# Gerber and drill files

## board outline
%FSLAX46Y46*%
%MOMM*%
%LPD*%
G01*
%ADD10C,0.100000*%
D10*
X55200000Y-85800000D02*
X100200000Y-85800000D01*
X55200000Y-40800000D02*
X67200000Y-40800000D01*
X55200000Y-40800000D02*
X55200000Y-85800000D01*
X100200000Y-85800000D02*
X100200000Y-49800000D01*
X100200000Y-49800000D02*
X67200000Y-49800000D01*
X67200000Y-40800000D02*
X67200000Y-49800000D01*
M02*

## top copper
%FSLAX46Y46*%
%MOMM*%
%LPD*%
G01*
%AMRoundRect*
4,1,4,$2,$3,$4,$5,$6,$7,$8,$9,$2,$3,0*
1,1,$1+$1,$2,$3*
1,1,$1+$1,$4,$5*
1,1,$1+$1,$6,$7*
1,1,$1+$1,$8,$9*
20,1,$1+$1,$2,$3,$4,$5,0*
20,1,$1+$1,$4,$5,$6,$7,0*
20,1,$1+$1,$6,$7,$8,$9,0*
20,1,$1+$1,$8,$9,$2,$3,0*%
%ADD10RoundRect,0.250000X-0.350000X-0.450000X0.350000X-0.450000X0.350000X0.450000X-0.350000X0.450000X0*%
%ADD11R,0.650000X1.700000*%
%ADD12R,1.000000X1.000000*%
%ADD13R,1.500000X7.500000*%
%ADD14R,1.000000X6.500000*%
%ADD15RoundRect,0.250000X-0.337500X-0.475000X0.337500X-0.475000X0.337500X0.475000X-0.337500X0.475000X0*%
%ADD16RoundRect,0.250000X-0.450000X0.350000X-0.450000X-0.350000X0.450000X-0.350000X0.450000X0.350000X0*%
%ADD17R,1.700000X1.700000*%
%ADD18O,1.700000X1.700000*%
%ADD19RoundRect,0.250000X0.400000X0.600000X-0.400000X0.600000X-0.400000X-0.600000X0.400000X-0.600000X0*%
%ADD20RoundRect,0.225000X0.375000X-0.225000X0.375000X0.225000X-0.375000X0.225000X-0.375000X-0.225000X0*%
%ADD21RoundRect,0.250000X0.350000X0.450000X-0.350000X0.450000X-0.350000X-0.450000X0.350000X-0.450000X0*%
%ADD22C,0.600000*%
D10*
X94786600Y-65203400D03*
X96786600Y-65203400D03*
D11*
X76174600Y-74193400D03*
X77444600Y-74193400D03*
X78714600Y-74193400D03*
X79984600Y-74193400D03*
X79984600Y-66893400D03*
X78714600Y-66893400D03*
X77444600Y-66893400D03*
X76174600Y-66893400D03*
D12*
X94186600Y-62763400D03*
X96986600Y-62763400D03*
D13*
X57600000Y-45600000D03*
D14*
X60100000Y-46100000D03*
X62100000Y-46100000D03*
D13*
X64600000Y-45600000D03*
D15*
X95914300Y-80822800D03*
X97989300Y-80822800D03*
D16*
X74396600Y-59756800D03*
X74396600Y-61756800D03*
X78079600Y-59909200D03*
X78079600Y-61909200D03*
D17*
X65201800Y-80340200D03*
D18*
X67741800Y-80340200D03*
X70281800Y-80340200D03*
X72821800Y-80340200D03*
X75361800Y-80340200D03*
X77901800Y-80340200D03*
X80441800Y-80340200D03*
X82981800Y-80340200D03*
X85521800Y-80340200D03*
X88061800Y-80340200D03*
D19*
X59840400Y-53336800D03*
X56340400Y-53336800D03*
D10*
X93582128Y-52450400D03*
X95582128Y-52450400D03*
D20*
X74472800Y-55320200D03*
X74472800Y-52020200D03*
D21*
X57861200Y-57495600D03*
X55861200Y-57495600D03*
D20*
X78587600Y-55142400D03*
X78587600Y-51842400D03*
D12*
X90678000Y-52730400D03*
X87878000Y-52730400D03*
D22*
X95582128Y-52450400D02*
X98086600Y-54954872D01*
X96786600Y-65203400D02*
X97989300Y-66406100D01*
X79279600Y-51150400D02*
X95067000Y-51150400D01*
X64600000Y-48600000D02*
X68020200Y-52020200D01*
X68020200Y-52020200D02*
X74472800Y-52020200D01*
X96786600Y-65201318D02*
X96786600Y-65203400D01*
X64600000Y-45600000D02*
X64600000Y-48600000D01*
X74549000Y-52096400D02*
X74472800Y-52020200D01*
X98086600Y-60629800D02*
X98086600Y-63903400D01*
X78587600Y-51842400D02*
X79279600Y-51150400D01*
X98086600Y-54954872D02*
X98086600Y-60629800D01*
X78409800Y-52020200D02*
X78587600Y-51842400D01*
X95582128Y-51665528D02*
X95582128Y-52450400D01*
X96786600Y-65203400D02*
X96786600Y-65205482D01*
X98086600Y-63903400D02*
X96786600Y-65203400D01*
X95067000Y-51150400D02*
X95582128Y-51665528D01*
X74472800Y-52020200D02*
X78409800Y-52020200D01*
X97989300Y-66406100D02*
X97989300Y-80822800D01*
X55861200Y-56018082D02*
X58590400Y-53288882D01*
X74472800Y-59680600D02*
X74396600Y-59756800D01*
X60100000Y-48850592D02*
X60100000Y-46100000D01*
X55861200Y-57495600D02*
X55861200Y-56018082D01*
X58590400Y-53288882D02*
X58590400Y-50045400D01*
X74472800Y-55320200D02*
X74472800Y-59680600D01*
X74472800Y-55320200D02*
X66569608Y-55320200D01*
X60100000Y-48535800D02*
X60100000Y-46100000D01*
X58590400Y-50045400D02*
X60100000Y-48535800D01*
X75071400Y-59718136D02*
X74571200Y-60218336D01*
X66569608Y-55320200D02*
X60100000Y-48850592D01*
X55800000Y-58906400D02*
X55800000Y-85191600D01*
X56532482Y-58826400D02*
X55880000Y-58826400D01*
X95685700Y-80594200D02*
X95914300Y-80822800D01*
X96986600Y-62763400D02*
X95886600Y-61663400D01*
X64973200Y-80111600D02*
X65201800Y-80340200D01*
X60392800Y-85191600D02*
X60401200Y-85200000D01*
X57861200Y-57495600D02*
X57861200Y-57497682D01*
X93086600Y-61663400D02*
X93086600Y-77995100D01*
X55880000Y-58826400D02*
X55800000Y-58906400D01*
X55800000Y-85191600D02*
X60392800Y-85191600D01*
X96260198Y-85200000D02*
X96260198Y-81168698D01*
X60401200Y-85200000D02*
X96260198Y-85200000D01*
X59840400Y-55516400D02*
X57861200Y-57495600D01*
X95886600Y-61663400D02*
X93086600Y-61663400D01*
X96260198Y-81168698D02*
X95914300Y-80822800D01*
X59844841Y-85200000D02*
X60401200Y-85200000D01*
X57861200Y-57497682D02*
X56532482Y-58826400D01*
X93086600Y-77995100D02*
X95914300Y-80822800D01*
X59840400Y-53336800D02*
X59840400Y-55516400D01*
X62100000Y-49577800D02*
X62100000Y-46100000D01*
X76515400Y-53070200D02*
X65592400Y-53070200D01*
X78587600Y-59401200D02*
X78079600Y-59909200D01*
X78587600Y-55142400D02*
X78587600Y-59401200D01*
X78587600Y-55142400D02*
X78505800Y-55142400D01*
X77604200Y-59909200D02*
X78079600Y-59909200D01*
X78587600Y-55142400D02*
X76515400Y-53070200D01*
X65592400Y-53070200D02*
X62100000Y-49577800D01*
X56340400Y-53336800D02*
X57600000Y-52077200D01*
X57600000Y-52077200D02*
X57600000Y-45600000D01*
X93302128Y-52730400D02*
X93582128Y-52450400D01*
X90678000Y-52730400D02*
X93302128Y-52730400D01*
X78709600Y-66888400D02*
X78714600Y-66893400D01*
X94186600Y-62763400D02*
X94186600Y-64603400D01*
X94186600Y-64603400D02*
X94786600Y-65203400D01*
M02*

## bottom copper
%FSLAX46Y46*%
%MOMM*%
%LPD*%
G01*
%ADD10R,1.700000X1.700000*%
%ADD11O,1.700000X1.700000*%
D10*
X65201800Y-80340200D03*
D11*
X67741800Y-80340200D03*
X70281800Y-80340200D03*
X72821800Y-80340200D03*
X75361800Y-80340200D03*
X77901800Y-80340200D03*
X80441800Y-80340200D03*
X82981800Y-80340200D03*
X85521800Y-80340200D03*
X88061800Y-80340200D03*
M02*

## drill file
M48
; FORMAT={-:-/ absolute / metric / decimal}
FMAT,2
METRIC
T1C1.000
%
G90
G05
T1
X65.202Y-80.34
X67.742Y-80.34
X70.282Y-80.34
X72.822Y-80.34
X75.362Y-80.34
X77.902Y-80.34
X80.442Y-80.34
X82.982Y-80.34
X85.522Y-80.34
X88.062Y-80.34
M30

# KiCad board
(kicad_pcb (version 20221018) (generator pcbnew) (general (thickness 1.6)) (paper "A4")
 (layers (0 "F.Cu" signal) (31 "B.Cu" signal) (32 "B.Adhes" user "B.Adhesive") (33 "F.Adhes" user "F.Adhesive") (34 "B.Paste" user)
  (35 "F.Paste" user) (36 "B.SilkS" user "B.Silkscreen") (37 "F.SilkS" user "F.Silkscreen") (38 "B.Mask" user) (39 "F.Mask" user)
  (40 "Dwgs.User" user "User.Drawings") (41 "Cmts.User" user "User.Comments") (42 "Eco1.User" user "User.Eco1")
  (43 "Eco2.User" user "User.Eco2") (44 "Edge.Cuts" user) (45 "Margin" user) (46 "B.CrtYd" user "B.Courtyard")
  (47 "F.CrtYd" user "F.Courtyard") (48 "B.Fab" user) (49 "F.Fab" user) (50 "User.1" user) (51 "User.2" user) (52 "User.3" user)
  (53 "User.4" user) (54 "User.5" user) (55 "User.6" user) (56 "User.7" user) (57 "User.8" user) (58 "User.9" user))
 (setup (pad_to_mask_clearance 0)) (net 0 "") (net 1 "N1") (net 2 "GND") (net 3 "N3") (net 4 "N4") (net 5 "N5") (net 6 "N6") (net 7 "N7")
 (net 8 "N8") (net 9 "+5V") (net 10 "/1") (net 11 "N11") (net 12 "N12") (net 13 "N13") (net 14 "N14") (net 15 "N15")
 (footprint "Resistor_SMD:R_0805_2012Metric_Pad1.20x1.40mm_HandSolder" (layer "F.Cu") (at 95.7866 65.2034)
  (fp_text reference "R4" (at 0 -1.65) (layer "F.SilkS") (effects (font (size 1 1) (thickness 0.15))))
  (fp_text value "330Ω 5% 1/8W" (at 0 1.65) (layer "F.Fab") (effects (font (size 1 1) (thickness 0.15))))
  (pad "1" smd roundrect (at -1 0) (size 1.2 1.4) (layers "F.Cu" "F.Paste" "F.Mask") (roundrect_rratio 0.208333) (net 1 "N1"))
  (pad "2" smd roundrect (at 1 0) (size 1.2 1.4) (layers "F.Cu" "F.Paste" "F.Mask") (roundrect_rratio 0.208333) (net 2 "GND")))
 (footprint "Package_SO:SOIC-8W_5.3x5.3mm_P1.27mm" (layer "F.Cu") (at 78.0796 70.5434 90)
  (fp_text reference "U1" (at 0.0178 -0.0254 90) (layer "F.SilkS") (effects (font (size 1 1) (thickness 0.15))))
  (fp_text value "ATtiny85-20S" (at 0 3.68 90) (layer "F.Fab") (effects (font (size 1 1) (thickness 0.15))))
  (pad "1" smd rect (at -3.65 -1.905 90) (size 1.7 0.65) (layers "F.Cu" "F.Paste" "F.Mask") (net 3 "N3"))
  (pad "2" smd rect (at -3.65 -0.635 90) (size 1.7 0.65) (layers "F.Cu" "F.Paste" "F.Mask") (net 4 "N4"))
  (pad "3" smd rect (at -3.65 0.635 90) (size 1.7 0.65) (layers "F.Cu" "F.Paste" "F.Mask") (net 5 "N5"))
  (pad "4" smd rect (at -3.65 1.905 90) (size 1.7 0.65) (layers "F.Cu" "F.Paste" "F.Mask") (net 2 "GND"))
  (pad "5" smd rect (at 3.65 1.905 90) (size 1.7 0.65) (layers "F.Cu" "F.Paste" "F.Mask") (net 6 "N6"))
  (pad "6" smd rect (at 3.65 0.635 90) (size 1.7 0.65) (layers "F.Cu" "F.Paste" "F.Mask") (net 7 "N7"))
  (pad "7" smd rect (at 3.65 -0.635 90) (size 1.7 0.65) (layers "F.Cu" "F.Paste" "F.Mask") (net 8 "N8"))
  (pad "8" smd rect (at 3.65 -1.905 90) (size 1.7 0.65) (layers "F.Cu" "F.Paste" "F.Mask") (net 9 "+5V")))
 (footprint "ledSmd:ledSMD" (layer "F.Cu") (at 95.9866 62.7634)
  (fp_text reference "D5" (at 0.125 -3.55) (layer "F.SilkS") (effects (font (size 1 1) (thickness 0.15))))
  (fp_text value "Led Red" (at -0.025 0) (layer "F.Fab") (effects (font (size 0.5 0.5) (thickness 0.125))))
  (pad "1" smd rect (at -1.8 0) (size 1 1) (layers "F.Cu" "F.Paste" "F.Mask") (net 1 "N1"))
  (pad "2" smd rect (at 1 0) (size 1 1) (layers "F.Cu" "F.Paste" "F.Mask") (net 9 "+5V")))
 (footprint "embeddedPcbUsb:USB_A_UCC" (layer "F.Cu") (at 61.1 45.8 -90)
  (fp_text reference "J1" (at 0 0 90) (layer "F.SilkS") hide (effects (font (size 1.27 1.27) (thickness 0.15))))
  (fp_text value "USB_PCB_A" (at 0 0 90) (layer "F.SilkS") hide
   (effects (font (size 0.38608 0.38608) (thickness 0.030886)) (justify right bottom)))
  (pad "1" smd rect (at -0.2 3.5 270) (size 7.5 1.5) (layers "F.Cu" "F.Paste" "F.Mask") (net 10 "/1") (solder_mask_margin 0.1016))
  (pad "2" smd rect (at 0.3 1 270) (size 6.5 1) (layers "F.Cu" "F.Paste" "F.Mask") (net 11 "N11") (solder_mask_margin 0.1016))
  (pad "3" smd rect (at 0.3 -1 270) (size 6.5 1) (layers "F.Cu" "F.Paste" "F.Mask") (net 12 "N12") (solder_mask_margin 0.1016))
  (pad "4" smd rect (at -0.2 -3.5 270) (size 7.5 1.5) (layers "F.Cu" "F.Paste" "F.Mask") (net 2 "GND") (solder_mask_margin 0.1016)))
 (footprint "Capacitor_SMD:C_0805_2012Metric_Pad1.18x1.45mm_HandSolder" (layer "F.Cu") (at 96.9518 80.8228)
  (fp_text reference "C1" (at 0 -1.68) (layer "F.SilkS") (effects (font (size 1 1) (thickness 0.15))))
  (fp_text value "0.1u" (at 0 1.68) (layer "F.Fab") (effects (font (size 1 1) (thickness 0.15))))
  (pad "1" smd roundrect (at -1.0375 0) (size 1.175 1.45) (layers "F.Cu" "F.Paste" "F.Mask") (roundrect_rratio 0.212766) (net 9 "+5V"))
  (pad "2" smd roundrect (at 1.0375 0) (size 1.175 1.45) (layers "F.Cu" "F.Paste" "F.Mask") (roundrect_rratio 0.212766) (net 2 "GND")))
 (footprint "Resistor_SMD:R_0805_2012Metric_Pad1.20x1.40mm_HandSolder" (layer "F.Cu") (at 74.3966 60.7568 -90)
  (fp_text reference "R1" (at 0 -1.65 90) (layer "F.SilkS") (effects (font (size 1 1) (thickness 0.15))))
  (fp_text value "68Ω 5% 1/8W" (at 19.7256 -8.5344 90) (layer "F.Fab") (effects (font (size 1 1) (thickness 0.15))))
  (pad "1" smd roundrect (at -1 0 270) (size 1.2 1.4) (layers "F.Cu" "F.Paste" "F.Mask") (roundrect_rratio 0.208333) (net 11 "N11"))
  (pad "2" smd roundrect (at 1 0 270) (size 1.2 1.4) (layers "F.Cu" "F.Paste" "F.Mask") (roundrect_rratio 0.208333) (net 4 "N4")))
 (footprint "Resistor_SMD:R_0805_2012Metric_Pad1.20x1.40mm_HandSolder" (layer "F.Cu") (at 78.0796 60.9092 -90)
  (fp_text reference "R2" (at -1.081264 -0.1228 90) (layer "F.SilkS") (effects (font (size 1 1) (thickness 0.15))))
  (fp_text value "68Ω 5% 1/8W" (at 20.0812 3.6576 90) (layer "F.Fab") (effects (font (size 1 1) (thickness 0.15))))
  (pad "1" smd roundrect (at -1 0 270) (size 1.2 1.4) (layers "F.Cu" "F.Paste" "F.Mask") (roundrect_rratio 0.208333) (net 12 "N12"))
  (pad "2" smd roundrect (at 1 0 270) (size 1.2 1.4) (layers "F.Cu" "F.Paste" "F.Mask") (roundrect_rratio 0.208333) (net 5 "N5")))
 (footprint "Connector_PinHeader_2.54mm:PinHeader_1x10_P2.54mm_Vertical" (layer "F.Cu") (at 65.2018 80.3402 90)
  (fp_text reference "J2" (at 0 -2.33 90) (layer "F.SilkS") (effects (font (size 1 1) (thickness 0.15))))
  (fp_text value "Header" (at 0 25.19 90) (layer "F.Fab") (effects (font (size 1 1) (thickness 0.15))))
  (pad "1" thru_hole rect (at 0 0 90) (size 1.7 1.7) (drill 1) (layers "*.Cu" "*.Mask") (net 9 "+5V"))
  (pad "2" thru_hole oval (at 0 2.54 90) (size 1.7 1.7) (drill 1) (layers "*.Cu" "*.Mask") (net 2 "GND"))
  (pad "3" thru_hole oval (at 0 5.08 90) (size 1.7 1.7) (drill 1) (layers "*.Cu" "*.Mask") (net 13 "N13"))
  (pad "4" thru_hole oval (at 0 7.62 90) (size 1.7 1.7) (drill 1) (layers "*.Cu" "*.Mask") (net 6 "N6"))
  (pad "5" thru_hole oval (at 0 10.16 90) (size 1.7 1.7) (drill 1) (layers "*.Cu" "*.Mask") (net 7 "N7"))
  (pad "6" thru_hole oval (at 0 12.7 90) (size 1.7 1.7) (drill 1) (layers "*.Cu" "*.Mask") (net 8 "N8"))
  (pad "7" thru_hole oval (at 0 15.24 90) (size 1.7 1.7) (drill 1) (layers "*.Cu" "*.Mask") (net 4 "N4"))
  (pad "8" thru_hole oval (at 0 17.78 90) (size 1.7 1.7) (drill 1) (layers "*.Cu" "*.Mask") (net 5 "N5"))
  (pad "9" thru_hole oval (at 0 20.32 90) (size 1.7 1.7) (drill 1) (layers "*.Cu" "*.Mask") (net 3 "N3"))
  (pad "10" thru_hole oval (at 0 22.86 90) (size 1.7 1.7) (drill 1) (layers "*.Cu" "*.Mask") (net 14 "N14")))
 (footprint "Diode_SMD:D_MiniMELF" (layer "F.Cu") (at 58.0904 53.3368 180)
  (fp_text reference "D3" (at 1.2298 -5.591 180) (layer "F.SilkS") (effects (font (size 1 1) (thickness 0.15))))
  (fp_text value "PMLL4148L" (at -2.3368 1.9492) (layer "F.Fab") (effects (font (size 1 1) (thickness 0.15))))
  (pad "1" smd roundrect (at -1.75 0 180) (size 1.3 1.7) (layers "F.Cu" "F.Paste" "F.Mask") (roundrect_rratio 0.1923076923) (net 9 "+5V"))
  (pad "2" smd roundrect (at 1.75 0 180) (size 1.3 1.7) (layers "F.Cu" "F.Paste" "F.Mask") (roundrect_rratio 0.1923076923) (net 10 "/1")))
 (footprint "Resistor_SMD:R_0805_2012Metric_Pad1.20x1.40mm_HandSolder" (layer "F.Cu") (at 94.582128 52.4504)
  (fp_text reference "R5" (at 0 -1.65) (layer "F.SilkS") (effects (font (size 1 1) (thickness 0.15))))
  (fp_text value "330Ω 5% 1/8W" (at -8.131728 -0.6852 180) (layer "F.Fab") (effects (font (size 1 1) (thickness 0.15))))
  (pad "1" smd roundrect (at -1 0) (size 1.2 1.4) (layers "F.Cu" "F.Paste" "F.Mask") (roundrect_rratio 0.208333) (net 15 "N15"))
  (pad "2" smd roundrect (at 1 0) (size 1.2 1.4) (layers "F.Cu" "F.Paste" "F.Mask") (roundrect_rratio 0.208333) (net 2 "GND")))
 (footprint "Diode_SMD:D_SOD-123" (layer "F.Cu") (at 74.4728 53.6702 90)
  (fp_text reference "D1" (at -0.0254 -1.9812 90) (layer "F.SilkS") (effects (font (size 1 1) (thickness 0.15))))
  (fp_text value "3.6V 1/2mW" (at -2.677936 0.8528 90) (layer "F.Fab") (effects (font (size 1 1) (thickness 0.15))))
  (pad "1" smd roundrect (at -1.65 0 90) (size 0.9 1.2) (layers "F.Cu" "F.Paste" "F.Mask") (roundrect_rratio 0.25) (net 11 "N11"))
  (pad "2" smd roundrect (at 1.65 0 90) (size 0.9 1.2) (layers "F.Cu" "F.Paste" "F.Mask") (roundrect_rratio 0.25) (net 2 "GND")))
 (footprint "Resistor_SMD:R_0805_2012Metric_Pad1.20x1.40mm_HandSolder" (layer "F.Cu") (at 56.8612 57.4956 180)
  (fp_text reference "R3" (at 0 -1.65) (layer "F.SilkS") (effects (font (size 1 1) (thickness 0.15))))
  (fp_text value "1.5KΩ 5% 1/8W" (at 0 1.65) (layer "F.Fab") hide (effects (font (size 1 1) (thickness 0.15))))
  (pad "1" smd roundrect (at -1 0 180) (size 1.2 1.4) (layers "F.Cu" "F.Paste" "F.Mask") (roundrect_rratio 0.208333) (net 9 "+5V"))
  (pad "2" smd roundrect (at 1 0 180) (size 1.2 1.4) (layers "F.Cu" "F.Paste" "F.Mask") (roundrect_rratio 0.208333) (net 11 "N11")))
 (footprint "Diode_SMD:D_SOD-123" (layer "F.Cu") (at 78.5876 53.4924 90)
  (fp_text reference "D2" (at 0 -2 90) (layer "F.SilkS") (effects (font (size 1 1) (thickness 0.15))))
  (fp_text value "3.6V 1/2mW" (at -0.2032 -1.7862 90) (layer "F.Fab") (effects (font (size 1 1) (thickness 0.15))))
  (pad "1" smd roundrect (at -1.65 0 90) (size 0.9 1.2) (layers "F.Cu" "F.Paste" "F.Mask") (roundrect_rratio 0.25) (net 12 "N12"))
  (pad "2" smd roundrect (at 1.65 0 90) (size 0.9 1.2) (layers "F.Cu" "F.Paste" "F.Mask") (roundrect_rratio 0.25) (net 2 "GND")))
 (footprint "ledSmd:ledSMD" (layer "F.Cu") (at 88.878 52.7304 180)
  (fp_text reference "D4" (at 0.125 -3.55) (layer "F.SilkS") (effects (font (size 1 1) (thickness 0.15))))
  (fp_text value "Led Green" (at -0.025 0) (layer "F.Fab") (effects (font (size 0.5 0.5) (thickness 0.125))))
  (pad "1" smd rect (at -1.8 0 180) (size 1 1) (layers "F.Cu" "F.Paste" "F.Mask") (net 15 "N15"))
  (pad "2" smd rect (at 1 0 180) (size 1 1) (layers "F.Cu" "F.Paste" "F.Mask") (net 7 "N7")))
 (gr_line (start 55.2 85.8) (end 100.2 85.8) (stroke (width 0.1) (type default)) (layer "Edge.Cuts"))
 (gr_line (start 55.2 40.8) (end 67.2 40.8) (stroke (width 0.1) (type default)) (layer "Edge.Cuts"))
 (gr_line (start 55.2 40.8) (end 55.2 85.8) (stroke (width 0.1) (type default)) (layer "Edge.Cuts"))
 (gr_line (start 100.2 85.8) (end 100.2 49.8) (stroke (width 0.1) (type default)) (layer "Edge.Cuts"))
 (gr_line (start 100.2 49.8) (end 67.2 49.8) (stroke (width 0.1) (type default)) (layer "Edge.Cuts"))
 (gr_line (start 67.2 40.8) (end 67.2 49.8) (stroke (width 0.1) (type default)) (layer "Edge.Cuts"))
 (segment (start 95.582128 52.4504) (end 98.0866 54.954872) (width 0.6) (layer "F.Cu") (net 2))
 (segment (start 96.7866 65.2034) (end 97.9893 66.4061) (width 0.6) (layer "F.Cu") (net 2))
 (segment (start 79.2796 51.1504) (end 95.067 51.1504) (width 0.6) (layer "F.Cu") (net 2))
 (segment (start 64.6 48.6) (end 68.0202 52.0202) (width 0.6) (layer "F.Cu") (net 2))
 (segment (start 68.0202 52.0202) (end 74.4728 52.0202) (width 0.6) (layer "F.Cu") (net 2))
 (segment (start 96.7866 65.201318) (end 96.7866 65.2034) (width 0.6) (layer "F.Cu") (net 2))
 (segment (start 64.6 45.6) (end 64.6 48.6) (width 0.6) (layer "F.Cu") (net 2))
 (segment (start 74.549 52.0964) (end 74.4728 52.0202) (width 0.6) (layer "F.Cu") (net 2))
 (segment (start 98.0866 60.6298) (end 98.0866 63.9034) (width 0.6) (layer "F.Cu") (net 2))
 (segment (start 78.5876 51.8424) (end 79.2796 51.1504) (width 0.6) (layer "F.Cu") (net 2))
 (segment (start 98.0866 54.954872) (end 98.0866 60.6298) (width 0.6) (layer "F.Cu") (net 2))
 (segment (start 78.4098 52.0202) (end 78.5876 51.8424) (width 0.6) (layer "F.Cu") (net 2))
 (segment (start 95.582128 51.665528) (end 95.582128 52.4504) (width 0.6) (layer "F.Cu") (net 2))
 (segment (start 96.7866 65.2034) (end 96.7866 65.205482) (width 0.6) (layer "F.Cu") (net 2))
 (segment (start 98.0866 63.9034) (end 96.7866 65.2034) (width 0.6) (layer "F.Cu") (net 2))
 (segment (start 95.067 51.1504) (end 95.582128 51.665528) (width 0.6) (layer "F.Cu") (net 2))
 (segment (start 74.4728 52.0202) (end 78.4098 52.0202) (width 0.6) (layer "F.Cu") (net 2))
 (segment (start 97.9893 66.4061) (end 97.9893 80.8228) (width 0.6) (layer "F.Cu") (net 2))
 (segment (start 55.8612 56.018082) (end 58.5904 53.288882) (width 0.6) (layer "F.Cu") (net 11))
 (segment (start 74.4728 59.6806) (end 74.3966 59.7568) (width 0.6) (layer "F.Cu") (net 11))
 (segment (start 60.1 48.850592) (end 60.1 46.1) (width 0.6) (layer "F.Cu") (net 11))
 (segment (start 55.8612 57.4956) (end 55.8612 56.018082) (width 0.6) (layer "F.Cu") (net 11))
 (segment (start 58.5904 53.288882) (end 58.5904 50.0454) (width 0.6) (layer "F.Cu") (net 11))
 (segment (start 74.4728 55.3202) (end 74.4728 59.6806) (width 0.6) (layer "F.Cu") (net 11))
 (segment (start 74.4728 55.3202) (end 66.569608 55.3202) (width 0.6) (layer "F.Cu") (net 11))
 (segment (start 60.1 48.5358) (end 60.1 46.1) (width 0.6) (layer "F.Cu") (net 11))
 (segment (start 58.5904 50.0454) (end 60.1 48.5358) (width 0.6) (layer "F.Cu") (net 11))
 (segment (start 75.0714 59.718136) (end 74.5712 60.218336) (width 0.6) (layer "F.Cu") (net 11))
 (segment (start 66.569608 55.3202) (end 60.1 48.850592) (width 0.6) (layer "F.Cu") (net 11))
 (segment (start 55.8 58.9064) (end 55.8 85.1916) (width 0.6) (layer "F.Cu") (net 9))
 (segment (start 56.532482 58.8264) (end 55.88 58.8264) (width 0.6) (layer "F.Cu") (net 9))
 (segment (start 95.6857 80.5942) (end 95.9143 80.8228) (width 0.6) (layer "F.Cu") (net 9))
 (segment (start 96.9866 62.7634) (end 95.8866 61.6634) (width 0.6) (layer "F.Cu") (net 9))
 (segment (start 64.9732 80.1116) (end 65.2018 80.3402) (width 0.6) (layer "F.Cu") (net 9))
 (segment (start 60.3928 85.1916) (end 60.4012 85.2) (width 0.6) (layer "F.Cu") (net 9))
 (segment (start 57.8612 57.4956) (end 57.8612 57.497682) (width 0.6) (layer "F.Cu") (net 9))
 (segment (start 93.0866 61.6634) (end 93.0866 77.9951) (width 0.6) (layer "F.Cu") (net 9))
 (segment (start 55.88 58.8264) (end 55.8 58.9064) (width 0.6) (layer "F.Cu") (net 9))
 (segment (start 55.8 85.1916) (end 60.3928 85.1916) (width 0.6) (layer "F.Cu") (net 9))
 (segment (start 96.260198 85.2) (end 96.260198 81.168698) (width 0.6) (layer "F.Cu") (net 9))
 (segment (start 60.4012 85.2) (end 96.260198 85.2) (width 0.6) (layer "F.Cu") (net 9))
 (segment (start 59.8404 55.5164) (end 57.8612 57.4956) (width 0.6) (layer "F.Cu") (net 9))
 (segment (start 95.8866 61.6634) (end 93.0866 61.6634) (width 0.6) (layer "F.Cu") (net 9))
 (segment (start 96.260198 81.168698) (end 95.9143 80.8228) (width 0.6) (layer "F.Cu") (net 9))
 (segment (start 59.844841 85.2) (end 60.4012 85.2) (width 0.6) (layer "F.Cu") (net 9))
 (segment (start 57.8612 57.497682) (end 56.532482 58.8264) (width 0.6) (layer "F.Cu") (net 9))
 (segment (start 93.0866 77.9951) (end 95.9143 80.8228) (width 0.6) (layer "F.Cu") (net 9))
 (segment (start 59.8404 53.3368) (end 59.8404 55.5164) (width 0.6) (layer "F.Cu") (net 9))
 (segment (start 62.1 49.5778) (end 62.1 46.1) (width 0.6) (layer "F.Cu") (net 12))
 (segment (start 76.5154 53.0702) (end 65.5924 53.0702) (width 0.6) (layer "F.Cu") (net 12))
 (segment (start 78.5876 59.4012) (end 78.0796 59.9092) (width 0.6) (layer "F.Cu") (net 12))
 (segment (start 78.5876 55.1424) (end 78.5876 59.4012) (width 0.6) (layer "F.Cu") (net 12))
 (segment (start 78.5876 55.1424) (end 78.5058 55.1424) (width 0.6) (layer "F.Cu") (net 12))
 (segment (start 77.6042 59.9092) (end 78.0796 59.9092) (width 0.6) (layer "F.Cu") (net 12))
 (segment (start 78.5876 55.1424) (end 76.5154 53.0702) (width 0.6) (layer "F.Cu") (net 12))
 (segment (start 65.5924 53.0702) (end 62.1 49.5778) (width 0.6) (layer "F.Cu") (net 12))
 (segment (start 56.3404 53.3368) (end 57.6 52.0772) (width 0.6) (layer "F.Cu") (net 10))
 (segment (start 57.6 52.0772) (end 57.6 45.6) (width 0.6) (layer "F.Cu") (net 10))
 (segment (start 93.302128 52.7304) (end 93.582128 52.4504) (width 0.6) (layer "F.Cu") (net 15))
 (segment (start 90.678 52.7304) (end 93.302128 52.7304) (width 0.6) (layer "F.Cu") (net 15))
 (segment (start 78.7096 66.8884) (end 78.7146 66.8934) (width 0.6) (layer "F.Cu") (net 7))
 (segment (start 94.1866 62.7634) (end 94.1866 64.6034) (width 0.6) (layer "F.Cu") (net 1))
 (segment (start 94.1866 64.6034) (end 94.7866 65.2034) (width 0.6) (layer "F.Cu") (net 1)))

